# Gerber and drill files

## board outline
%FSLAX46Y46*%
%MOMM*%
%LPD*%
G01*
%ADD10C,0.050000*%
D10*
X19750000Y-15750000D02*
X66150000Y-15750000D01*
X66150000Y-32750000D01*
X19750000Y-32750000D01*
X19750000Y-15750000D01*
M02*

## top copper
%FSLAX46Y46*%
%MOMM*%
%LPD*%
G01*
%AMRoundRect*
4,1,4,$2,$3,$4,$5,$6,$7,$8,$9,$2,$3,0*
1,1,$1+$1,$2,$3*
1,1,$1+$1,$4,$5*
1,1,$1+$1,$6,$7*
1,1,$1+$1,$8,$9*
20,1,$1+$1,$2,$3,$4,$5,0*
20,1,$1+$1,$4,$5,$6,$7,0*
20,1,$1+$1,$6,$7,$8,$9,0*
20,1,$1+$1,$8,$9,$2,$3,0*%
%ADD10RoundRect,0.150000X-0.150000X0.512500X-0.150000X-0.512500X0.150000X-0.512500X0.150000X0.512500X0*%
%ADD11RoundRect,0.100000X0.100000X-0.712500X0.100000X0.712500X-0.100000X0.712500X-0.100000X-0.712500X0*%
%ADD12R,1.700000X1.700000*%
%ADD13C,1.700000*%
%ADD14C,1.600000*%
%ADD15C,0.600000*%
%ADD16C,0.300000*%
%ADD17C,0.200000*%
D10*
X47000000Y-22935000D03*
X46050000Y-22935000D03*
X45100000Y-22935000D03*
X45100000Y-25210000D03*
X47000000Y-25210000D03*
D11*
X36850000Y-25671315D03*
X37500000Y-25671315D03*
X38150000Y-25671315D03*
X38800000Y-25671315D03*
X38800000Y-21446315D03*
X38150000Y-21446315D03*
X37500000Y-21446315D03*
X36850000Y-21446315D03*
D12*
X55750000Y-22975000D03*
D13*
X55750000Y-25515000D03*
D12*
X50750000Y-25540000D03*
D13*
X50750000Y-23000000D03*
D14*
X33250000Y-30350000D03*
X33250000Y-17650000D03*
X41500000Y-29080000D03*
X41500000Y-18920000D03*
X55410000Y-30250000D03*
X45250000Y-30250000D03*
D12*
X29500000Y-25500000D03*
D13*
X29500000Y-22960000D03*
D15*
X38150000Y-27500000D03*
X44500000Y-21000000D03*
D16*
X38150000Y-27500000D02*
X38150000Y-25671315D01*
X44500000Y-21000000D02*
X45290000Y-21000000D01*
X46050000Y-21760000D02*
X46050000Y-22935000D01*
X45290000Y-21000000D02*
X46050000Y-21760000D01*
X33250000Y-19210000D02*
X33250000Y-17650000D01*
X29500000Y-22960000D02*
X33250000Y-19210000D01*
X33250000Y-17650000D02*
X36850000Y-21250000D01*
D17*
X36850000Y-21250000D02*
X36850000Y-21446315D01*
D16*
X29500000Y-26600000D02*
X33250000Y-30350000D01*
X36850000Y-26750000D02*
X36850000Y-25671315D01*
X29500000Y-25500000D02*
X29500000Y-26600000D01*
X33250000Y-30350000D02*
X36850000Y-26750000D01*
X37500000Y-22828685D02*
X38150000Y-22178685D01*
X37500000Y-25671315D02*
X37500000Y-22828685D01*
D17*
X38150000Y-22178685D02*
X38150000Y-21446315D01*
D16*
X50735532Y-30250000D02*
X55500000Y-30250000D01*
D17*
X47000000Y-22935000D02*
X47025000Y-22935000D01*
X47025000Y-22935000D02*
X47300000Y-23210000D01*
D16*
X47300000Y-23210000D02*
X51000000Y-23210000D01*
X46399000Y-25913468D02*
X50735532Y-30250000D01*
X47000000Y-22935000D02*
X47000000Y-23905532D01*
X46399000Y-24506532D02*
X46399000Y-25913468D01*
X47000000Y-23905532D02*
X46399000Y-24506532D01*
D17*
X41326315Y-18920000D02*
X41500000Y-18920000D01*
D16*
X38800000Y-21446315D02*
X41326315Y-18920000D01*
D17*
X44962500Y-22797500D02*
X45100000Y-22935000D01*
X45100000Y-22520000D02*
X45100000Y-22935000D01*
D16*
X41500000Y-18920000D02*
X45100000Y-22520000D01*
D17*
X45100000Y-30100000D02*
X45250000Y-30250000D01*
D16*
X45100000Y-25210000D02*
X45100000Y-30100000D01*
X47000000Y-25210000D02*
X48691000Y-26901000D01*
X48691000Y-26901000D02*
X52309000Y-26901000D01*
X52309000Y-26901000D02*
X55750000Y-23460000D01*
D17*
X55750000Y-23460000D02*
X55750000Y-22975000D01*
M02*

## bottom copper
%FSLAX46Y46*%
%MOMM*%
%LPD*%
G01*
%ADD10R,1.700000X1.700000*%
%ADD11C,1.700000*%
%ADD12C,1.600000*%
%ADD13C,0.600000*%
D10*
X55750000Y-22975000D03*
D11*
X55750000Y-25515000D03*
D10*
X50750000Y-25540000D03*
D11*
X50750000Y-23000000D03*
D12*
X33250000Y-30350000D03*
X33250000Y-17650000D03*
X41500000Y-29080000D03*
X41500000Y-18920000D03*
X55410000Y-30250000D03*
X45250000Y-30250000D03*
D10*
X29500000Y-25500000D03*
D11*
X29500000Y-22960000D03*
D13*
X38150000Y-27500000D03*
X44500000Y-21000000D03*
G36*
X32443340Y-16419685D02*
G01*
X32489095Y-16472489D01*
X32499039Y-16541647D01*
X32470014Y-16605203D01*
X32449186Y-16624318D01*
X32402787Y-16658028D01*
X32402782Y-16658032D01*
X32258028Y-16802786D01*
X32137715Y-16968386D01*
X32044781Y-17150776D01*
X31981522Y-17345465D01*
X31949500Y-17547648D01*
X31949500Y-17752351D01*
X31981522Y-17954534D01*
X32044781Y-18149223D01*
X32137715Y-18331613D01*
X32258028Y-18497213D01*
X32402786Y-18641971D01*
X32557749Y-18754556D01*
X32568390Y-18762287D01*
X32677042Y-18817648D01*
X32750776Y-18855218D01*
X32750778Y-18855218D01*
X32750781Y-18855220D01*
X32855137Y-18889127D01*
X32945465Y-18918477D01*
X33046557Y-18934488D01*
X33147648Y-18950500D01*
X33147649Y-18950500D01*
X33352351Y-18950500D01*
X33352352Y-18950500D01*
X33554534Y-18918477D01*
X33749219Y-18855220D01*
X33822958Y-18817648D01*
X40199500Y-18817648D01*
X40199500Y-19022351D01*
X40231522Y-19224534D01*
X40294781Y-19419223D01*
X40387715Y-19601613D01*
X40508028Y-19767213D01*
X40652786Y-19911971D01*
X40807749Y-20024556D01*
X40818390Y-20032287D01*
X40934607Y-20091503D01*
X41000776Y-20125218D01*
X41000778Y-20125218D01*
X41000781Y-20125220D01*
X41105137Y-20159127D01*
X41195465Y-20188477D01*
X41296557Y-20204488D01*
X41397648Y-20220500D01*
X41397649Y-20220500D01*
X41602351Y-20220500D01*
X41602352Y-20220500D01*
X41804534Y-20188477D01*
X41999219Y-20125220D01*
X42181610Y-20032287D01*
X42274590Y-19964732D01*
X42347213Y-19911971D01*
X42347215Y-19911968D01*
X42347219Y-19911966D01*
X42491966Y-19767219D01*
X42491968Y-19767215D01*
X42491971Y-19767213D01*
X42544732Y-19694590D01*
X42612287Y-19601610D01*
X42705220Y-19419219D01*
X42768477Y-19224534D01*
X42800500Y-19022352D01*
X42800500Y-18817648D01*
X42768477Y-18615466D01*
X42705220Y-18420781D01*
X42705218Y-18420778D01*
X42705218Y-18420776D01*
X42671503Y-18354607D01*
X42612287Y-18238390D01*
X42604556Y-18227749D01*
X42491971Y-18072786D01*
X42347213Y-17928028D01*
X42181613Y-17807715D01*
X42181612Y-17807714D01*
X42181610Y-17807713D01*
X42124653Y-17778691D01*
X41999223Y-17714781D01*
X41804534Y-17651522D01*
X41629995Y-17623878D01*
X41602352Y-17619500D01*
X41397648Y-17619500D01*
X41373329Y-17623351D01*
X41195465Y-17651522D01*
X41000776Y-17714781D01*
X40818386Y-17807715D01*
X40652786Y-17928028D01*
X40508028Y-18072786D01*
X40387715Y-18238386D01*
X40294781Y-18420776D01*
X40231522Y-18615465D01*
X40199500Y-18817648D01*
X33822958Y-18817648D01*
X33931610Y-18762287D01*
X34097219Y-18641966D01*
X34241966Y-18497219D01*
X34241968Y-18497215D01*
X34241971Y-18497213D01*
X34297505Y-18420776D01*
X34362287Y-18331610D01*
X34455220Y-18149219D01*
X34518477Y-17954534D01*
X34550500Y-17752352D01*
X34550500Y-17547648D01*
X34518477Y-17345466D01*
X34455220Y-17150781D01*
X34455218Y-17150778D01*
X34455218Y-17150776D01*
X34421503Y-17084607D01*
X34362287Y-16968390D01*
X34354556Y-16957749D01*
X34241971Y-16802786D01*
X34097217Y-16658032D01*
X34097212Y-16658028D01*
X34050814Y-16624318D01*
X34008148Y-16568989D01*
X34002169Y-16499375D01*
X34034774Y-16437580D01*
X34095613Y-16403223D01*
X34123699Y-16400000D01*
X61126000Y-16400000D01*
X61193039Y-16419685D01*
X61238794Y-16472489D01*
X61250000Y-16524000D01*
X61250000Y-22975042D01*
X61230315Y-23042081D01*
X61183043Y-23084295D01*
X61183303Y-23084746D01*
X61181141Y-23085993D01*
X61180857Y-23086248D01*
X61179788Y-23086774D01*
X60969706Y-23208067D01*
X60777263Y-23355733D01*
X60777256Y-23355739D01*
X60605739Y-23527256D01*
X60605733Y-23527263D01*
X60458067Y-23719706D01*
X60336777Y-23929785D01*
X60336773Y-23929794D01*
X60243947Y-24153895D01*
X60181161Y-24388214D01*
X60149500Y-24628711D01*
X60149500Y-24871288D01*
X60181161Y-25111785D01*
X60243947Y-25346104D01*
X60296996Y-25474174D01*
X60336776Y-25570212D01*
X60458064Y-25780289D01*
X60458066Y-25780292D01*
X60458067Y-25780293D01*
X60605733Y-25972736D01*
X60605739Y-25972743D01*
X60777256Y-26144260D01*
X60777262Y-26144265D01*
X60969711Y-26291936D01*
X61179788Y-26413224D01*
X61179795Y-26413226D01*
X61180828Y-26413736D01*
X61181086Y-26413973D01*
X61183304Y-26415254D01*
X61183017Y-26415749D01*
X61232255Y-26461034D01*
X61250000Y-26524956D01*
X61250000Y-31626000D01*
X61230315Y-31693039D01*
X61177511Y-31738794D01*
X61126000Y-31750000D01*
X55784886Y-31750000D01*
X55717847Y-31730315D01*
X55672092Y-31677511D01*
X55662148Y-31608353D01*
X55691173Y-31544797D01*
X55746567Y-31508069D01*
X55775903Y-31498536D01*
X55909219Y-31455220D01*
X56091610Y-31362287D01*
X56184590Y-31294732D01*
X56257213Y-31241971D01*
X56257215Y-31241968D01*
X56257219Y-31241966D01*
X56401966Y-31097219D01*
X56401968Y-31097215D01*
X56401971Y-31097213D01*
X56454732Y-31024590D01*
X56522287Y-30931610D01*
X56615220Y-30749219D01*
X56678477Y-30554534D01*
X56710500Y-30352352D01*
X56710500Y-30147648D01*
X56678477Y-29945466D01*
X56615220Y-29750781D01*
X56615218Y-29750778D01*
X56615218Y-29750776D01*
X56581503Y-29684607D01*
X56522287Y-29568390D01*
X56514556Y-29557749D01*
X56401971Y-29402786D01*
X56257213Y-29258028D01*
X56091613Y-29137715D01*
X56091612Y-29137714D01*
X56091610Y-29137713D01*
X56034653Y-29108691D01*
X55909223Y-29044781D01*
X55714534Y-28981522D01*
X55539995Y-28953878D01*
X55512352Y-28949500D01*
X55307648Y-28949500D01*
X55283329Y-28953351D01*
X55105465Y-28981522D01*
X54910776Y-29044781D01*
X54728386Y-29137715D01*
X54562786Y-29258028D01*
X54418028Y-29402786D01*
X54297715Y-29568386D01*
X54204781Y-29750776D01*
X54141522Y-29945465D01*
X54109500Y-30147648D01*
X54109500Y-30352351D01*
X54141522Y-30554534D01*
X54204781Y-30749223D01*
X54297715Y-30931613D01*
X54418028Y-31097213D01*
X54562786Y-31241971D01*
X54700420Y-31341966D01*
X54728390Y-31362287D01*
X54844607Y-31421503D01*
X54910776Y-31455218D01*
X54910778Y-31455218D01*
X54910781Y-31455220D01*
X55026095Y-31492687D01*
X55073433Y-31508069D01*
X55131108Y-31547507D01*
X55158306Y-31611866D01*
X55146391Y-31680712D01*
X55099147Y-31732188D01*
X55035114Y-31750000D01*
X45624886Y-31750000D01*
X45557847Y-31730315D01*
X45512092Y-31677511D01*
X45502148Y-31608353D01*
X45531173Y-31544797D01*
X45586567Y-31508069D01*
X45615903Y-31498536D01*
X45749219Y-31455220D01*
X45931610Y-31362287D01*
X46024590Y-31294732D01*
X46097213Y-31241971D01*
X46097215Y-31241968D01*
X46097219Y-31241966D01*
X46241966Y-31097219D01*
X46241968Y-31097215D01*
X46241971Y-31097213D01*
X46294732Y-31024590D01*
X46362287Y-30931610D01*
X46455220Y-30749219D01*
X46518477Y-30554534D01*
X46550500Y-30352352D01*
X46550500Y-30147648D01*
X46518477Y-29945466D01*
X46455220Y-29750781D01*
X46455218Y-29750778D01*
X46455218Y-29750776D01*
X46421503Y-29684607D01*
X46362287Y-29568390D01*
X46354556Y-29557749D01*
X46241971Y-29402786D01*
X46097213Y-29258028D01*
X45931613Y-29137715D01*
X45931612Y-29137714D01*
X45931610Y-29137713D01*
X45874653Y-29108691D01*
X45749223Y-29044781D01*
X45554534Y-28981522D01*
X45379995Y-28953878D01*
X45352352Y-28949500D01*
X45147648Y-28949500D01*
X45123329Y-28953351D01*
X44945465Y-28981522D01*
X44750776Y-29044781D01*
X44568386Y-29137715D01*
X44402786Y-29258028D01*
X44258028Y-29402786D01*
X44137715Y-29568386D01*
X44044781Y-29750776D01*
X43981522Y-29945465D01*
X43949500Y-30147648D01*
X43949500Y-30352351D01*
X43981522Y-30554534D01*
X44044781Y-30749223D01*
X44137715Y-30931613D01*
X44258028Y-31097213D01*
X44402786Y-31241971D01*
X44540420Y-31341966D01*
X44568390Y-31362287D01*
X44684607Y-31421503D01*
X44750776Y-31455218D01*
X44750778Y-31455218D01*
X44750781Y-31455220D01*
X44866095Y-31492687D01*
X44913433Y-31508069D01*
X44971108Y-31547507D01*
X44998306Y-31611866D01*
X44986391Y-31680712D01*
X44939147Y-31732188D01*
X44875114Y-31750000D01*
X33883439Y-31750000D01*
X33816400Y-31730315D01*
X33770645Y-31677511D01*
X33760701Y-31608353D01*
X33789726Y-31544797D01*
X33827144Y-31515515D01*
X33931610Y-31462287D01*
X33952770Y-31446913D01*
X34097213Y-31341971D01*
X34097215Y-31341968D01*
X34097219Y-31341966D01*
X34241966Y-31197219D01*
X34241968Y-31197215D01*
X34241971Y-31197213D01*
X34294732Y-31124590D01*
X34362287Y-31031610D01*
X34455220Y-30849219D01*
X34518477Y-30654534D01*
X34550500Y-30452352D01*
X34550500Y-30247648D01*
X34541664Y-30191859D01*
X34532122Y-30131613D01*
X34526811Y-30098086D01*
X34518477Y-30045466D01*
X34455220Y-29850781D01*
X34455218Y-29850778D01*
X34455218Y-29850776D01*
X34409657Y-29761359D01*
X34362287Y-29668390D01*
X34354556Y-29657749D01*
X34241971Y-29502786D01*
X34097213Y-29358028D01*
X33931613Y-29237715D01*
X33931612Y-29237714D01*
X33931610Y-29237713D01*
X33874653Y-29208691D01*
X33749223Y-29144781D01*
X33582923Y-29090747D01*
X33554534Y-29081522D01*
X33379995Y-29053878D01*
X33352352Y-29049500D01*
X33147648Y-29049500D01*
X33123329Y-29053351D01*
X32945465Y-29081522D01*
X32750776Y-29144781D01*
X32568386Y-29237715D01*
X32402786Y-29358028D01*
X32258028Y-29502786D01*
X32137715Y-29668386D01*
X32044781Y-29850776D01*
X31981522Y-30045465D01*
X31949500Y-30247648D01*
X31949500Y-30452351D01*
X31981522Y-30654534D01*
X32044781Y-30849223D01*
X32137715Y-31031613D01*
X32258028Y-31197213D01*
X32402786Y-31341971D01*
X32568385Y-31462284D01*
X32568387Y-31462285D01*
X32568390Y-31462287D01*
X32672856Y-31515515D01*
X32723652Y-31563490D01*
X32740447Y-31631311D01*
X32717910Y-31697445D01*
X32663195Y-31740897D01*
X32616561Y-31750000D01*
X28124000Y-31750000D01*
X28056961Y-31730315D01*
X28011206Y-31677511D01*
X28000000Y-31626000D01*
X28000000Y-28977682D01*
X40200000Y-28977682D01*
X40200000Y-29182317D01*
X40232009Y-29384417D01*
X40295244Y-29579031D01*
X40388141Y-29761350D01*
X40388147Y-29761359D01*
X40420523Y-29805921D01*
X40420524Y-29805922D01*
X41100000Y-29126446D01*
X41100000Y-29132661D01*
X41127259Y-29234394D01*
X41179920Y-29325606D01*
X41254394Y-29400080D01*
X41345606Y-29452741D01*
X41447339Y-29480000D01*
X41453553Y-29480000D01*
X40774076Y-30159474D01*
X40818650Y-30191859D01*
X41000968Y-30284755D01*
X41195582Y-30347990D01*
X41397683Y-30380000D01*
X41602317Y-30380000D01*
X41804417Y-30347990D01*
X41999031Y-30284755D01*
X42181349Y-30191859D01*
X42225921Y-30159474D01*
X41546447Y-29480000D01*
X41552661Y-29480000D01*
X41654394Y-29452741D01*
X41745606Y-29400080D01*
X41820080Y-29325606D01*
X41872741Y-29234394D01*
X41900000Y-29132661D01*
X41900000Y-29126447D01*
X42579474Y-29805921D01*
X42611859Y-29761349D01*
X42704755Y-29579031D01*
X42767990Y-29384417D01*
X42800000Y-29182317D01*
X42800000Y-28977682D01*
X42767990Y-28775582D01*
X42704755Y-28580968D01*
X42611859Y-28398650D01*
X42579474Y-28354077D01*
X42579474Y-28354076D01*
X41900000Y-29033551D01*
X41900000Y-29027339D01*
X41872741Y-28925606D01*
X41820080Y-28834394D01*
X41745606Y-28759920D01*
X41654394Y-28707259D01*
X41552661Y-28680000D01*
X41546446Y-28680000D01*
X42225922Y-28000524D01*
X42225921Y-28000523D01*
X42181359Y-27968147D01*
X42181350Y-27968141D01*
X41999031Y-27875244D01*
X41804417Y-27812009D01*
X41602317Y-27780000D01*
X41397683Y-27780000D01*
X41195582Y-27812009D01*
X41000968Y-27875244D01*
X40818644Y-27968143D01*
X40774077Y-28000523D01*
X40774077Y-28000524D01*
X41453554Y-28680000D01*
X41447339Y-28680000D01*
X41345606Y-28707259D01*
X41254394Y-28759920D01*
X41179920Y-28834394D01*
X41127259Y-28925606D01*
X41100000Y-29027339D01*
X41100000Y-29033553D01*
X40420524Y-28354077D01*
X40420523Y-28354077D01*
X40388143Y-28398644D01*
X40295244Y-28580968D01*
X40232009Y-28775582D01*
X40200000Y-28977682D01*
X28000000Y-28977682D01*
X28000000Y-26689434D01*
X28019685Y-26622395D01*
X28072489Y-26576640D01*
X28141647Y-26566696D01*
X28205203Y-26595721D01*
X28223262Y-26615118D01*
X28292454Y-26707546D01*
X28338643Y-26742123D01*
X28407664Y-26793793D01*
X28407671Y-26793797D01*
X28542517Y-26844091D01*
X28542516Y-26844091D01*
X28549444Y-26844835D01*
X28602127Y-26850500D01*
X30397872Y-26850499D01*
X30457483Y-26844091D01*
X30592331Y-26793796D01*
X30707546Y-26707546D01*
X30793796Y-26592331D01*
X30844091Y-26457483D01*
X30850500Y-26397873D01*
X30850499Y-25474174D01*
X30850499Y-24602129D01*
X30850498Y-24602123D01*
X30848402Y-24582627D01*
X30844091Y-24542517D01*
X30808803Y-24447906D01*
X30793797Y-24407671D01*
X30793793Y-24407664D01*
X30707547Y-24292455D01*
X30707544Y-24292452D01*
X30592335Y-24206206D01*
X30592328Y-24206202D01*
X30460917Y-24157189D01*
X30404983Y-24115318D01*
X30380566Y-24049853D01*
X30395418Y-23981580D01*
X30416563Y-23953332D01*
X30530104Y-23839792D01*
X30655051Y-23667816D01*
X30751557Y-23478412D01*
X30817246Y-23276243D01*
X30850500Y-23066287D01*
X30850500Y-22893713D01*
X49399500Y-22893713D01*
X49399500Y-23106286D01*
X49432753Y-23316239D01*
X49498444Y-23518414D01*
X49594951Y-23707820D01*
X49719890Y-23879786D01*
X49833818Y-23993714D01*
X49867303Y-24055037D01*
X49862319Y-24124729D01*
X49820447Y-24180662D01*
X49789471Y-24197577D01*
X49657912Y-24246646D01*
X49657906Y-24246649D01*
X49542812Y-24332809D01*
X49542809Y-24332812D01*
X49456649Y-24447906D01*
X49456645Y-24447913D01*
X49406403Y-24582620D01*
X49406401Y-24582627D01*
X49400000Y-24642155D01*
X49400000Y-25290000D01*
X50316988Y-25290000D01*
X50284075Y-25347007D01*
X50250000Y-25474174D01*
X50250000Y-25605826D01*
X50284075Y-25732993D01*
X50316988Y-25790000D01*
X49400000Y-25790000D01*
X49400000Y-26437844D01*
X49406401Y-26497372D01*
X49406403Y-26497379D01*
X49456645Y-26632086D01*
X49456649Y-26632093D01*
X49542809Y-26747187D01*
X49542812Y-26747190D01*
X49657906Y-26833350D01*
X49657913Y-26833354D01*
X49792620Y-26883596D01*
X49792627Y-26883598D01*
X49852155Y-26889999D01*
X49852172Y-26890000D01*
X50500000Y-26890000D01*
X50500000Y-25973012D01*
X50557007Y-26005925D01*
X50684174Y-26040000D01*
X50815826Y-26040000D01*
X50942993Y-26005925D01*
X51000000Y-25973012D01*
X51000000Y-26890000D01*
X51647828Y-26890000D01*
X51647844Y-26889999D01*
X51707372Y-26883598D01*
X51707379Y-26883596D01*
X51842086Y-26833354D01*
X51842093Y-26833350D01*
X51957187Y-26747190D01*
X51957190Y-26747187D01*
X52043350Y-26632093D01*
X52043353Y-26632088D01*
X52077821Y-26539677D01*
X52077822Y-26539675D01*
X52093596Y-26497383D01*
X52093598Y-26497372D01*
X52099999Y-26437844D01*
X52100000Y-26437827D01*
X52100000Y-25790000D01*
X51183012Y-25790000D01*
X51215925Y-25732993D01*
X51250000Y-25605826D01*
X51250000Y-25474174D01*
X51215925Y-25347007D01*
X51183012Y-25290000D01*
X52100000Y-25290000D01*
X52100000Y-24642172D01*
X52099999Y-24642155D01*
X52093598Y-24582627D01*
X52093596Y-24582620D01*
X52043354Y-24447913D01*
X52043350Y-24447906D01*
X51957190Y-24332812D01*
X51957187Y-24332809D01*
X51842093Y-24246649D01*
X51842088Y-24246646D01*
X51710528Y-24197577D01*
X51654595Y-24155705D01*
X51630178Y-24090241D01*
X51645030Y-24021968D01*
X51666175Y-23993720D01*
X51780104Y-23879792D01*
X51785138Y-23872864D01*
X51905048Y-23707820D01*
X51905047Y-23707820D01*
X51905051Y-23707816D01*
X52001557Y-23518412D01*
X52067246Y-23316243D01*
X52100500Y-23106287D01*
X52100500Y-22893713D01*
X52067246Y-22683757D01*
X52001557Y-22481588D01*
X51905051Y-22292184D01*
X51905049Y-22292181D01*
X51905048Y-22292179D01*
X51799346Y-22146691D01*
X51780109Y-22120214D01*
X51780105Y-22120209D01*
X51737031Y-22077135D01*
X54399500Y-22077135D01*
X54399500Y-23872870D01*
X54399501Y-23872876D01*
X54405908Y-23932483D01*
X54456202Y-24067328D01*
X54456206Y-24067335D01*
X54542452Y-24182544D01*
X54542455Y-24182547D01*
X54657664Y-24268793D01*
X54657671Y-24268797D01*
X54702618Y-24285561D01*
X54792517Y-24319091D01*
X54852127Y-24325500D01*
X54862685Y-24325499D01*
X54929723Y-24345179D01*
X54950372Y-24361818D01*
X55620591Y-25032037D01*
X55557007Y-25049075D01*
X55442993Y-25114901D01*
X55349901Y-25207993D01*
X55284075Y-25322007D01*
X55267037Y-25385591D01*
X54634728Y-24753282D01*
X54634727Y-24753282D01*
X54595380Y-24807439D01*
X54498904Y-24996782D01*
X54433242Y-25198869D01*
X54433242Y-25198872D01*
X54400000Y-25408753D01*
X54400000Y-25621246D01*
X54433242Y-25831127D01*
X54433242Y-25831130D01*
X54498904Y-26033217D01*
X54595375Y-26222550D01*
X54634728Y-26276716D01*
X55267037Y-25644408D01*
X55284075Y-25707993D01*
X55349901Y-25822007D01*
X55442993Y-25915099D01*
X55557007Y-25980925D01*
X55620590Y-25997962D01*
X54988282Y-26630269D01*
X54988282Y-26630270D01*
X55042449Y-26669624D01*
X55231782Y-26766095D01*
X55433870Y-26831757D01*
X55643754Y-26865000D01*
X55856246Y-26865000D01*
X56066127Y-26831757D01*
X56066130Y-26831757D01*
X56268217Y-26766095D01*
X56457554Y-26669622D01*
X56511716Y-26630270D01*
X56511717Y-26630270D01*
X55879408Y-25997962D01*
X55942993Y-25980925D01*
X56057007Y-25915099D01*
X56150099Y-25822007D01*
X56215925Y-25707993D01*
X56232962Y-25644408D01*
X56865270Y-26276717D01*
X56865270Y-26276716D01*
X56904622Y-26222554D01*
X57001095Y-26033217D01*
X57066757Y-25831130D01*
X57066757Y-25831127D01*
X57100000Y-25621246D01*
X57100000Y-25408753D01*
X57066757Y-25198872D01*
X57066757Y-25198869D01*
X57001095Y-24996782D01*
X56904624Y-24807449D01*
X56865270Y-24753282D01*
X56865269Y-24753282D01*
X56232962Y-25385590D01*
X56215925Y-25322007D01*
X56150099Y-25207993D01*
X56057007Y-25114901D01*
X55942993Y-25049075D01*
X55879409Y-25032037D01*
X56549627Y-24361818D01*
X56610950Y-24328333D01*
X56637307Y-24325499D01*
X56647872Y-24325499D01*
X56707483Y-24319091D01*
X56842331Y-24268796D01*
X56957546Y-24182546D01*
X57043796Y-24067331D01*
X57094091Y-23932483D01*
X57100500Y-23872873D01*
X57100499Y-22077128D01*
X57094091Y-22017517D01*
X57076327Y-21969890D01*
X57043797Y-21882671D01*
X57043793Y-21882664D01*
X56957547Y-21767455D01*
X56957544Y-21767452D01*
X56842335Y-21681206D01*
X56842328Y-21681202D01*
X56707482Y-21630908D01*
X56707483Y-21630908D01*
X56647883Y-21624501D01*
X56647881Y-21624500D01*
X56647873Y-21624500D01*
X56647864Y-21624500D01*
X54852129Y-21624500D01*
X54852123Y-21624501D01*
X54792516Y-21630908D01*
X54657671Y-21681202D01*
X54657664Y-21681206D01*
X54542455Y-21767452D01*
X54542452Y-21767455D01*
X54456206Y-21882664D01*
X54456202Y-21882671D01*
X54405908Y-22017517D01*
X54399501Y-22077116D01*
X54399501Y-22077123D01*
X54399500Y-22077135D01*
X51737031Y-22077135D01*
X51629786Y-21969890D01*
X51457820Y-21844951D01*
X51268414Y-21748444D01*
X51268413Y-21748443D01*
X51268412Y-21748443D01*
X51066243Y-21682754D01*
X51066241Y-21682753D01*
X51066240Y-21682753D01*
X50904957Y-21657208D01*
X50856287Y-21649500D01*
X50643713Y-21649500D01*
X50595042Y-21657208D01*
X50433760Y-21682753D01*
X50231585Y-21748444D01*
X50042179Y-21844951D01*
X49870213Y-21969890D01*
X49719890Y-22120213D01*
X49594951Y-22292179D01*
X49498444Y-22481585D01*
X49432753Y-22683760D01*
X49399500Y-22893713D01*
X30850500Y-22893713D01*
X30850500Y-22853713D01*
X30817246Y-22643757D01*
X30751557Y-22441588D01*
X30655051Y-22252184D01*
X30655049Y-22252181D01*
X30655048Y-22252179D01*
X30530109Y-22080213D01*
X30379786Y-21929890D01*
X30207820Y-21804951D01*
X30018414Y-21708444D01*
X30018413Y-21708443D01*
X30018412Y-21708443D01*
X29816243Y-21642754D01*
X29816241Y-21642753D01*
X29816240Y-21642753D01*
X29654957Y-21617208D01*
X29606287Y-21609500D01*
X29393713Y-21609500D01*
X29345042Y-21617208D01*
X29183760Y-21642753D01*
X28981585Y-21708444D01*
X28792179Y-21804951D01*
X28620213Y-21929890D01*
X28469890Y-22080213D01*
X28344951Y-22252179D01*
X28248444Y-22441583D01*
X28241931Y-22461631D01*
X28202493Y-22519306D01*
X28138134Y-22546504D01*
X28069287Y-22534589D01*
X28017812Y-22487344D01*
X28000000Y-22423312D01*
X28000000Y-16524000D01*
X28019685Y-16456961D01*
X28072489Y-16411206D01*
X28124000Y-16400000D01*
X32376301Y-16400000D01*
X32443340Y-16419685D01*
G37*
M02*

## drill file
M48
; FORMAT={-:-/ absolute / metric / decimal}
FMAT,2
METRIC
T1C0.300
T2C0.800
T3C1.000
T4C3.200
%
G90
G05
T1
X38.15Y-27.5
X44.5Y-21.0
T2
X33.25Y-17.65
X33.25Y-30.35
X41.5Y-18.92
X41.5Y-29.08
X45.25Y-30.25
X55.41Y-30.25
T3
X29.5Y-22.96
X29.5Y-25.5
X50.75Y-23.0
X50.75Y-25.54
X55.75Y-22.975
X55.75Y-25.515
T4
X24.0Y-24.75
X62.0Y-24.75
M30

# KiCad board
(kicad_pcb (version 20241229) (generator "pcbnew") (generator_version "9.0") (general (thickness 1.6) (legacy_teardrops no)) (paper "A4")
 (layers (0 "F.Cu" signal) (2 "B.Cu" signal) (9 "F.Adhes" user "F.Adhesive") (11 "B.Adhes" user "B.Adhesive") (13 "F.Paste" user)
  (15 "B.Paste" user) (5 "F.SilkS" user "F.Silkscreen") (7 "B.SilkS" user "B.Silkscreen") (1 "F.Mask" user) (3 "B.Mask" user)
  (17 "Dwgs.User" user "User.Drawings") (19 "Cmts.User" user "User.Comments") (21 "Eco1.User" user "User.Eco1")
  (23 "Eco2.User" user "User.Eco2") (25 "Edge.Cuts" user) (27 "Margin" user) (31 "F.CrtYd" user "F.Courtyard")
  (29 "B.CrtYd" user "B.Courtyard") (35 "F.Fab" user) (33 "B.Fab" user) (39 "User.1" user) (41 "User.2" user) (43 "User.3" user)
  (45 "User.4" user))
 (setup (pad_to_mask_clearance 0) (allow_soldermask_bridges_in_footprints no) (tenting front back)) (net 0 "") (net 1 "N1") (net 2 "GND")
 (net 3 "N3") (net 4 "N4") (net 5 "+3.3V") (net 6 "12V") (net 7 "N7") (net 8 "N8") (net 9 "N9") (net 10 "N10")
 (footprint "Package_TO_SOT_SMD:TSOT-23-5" (layer "F.Cu") (at 46.05 24.0725 -90)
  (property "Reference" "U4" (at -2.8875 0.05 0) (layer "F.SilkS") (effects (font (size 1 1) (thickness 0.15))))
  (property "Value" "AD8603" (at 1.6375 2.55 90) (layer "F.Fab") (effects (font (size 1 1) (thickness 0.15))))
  (pad "1" smd roundrect (at -1.1375 -0.95 270) (size 1.325 0.6) (layers "F.Cu" "F.Mask" "F.Paste") (roundrect_rratio 0.25) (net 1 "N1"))
  (pad "2" smd roundrect (at -1.1375 0 270) (size 1.325 0.6) (layers "F.Cu" "F.Mask" "F.Paste") (roundrect_rratio 0.25) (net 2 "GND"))
  (pad "3" smd roundrect (at -1.1375 0.95 270) (size 1.325 0.6) (layers "F.Cu" "F.Mask" "F.Paste") (roundrect_rratio 0.25) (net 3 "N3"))
  (pad "4" smd roundrect (at 1.1375 0.95 270) (size 1.325 0.6) (layers "F.Cu" "F.Mask" "F.Paste") (roundrect_rratio 0.25) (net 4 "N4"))
  (pad "5" smd roundrect (at 1.1375 -0.95 270) (size 1.325 0.6) (layers "F.Cu" "F.Mask" "F.Paste") (roundrect_rratio 0.25) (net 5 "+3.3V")))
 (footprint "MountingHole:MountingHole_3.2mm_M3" (layer "F.Cu") (at 62 24.75)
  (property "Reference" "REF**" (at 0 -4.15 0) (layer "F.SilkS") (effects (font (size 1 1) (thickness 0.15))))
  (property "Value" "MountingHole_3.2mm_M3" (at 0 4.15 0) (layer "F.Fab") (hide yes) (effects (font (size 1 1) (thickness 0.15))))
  (pad "" np_thru_hole circle (at 0 0) (size 3.2 3.2) (drill 3.2) (layers "*.Cu" "*.Mask")))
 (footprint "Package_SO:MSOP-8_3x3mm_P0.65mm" (layer "F.Cu") (at 37.825 23.558815 90)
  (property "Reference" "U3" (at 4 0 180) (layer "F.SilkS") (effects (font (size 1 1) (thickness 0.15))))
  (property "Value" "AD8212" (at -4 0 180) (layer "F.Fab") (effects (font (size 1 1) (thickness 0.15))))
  (pad "1" smd roundrect (at -2.1125 -0.975 90) (size 1.625 0.4) (layers "F.Cu" "F.Mask" "F.Paste") (roundrect_rratio 0.25) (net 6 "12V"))
  (pad "2" smd roundrect (at -2.1125 -0.325 90) (size 1.625 0.4) (layers "F.Cu" "F.Mask" "F.Paste") (roundrect_rratio 0.25) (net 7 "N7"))
  (pad "3" smd roundrect (at -2.1125 0.325 90) (size 1.625 0.4) (layers "F.Cu" "F.Mask" "F.Paste") (roundrect_rratio 0.25) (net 2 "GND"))
  (pad "4" smd roundrect (at -2.1125 0.975 90) (size 1.625 0.4) (layers "F.Cu" "F.Mask" "F.Paste") (roundrect_rratio 0.25) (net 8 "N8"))
  (pad "5" smd roundrect (at 2.1125 0.975 90) (size 1.625 0.4) (layers "F.Cu" "F.Mask" "F.Paste") (roundrect_rratio 0.25) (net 3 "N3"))
  (pad "6" smd roundrect (at 2.1125 0.325 90) (size 1.625 0.4) (layers "F.Cu" "F.Mask" "F.Paste") (roundrect_rratio 0.25) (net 7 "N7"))
  (pad "7" smd roundrect (at 2.1125 -0.325 90) (size 1.625 0.4) (layers "F.Cu" "F.Mask" "F.Paste") (roundrect_rratio 0.25) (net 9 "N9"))
  (pad "8" smd roundrect (at 2.1125 -0.975 90) (size 1.625 0.4) (layers "F.Cu" "F.Mask" "F.Paste") (roundrect_rratio 0.25) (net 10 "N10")))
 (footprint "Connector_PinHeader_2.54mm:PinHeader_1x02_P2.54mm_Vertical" (layer "F.Cu") (at 55.75 22.975)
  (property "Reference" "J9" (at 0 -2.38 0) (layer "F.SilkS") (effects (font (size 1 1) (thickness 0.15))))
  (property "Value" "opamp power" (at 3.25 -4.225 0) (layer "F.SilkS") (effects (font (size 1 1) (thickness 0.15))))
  (pad "1" thru_hole rect (at 0 0) (size 1.7 1.7) (drill 1) (layers "*.Cu" "*.Mask") (remove_unused_layers no) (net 5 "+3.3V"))
  (pad "2" thru_hole circle (at 0 2.54) (size 1.7 1.7) (drill 1) (layers "*.Cu" "*.Mask") (remove_unused_layers no) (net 2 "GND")))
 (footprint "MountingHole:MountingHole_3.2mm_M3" (layer "F.Cu") (at 24 24.75)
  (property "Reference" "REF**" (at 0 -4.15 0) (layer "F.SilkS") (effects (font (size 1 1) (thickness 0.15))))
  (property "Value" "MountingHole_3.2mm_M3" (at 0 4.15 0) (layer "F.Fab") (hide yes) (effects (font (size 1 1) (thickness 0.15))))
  (pad "" np_thru_hole circle (at 0 0) (size 3.2 3.2) (drill 3.2) (layers "*.Cu" "*.Mask")))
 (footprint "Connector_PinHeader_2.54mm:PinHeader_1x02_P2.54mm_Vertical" (layer "F.Cu") (at 50.75 25.54 180)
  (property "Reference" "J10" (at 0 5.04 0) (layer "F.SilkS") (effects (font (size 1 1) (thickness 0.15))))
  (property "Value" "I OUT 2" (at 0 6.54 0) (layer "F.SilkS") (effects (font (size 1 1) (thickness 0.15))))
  (pad "1" thru_hole rect (at 0 0 180) (size 1.7 1.7) (drill 1) (layers "*.Cu" "*.Mask") (remove_unused_layers no) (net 2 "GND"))
  (pad "2" thru_hole circle (at 0 2.54 180) (size 1.7 1.7) (drill 1) (layers "*.Cu" "*.Mask") (remove_unused_layers no) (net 1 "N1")))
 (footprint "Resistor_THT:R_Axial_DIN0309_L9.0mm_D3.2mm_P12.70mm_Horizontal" (layer "F.Cu") (at 33.25 30.35 90)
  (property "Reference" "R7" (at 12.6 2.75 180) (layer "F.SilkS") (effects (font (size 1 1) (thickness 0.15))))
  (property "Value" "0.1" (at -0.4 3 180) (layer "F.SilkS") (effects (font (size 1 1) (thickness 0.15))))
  (pad "1" thru_hole circle (at 0 0 90) (size 1.6 1.6) (drill 0.8) (layers "*.Cu" "*.Mask") (remove_unused_layers no) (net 6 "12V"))
  (pad "2" thru_hole circle (at 12.7 0 90) (size 1.6 1.6) (drill 0.8) (layers "*.Cu" "*.Mask") (remove_unused_layers no) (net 10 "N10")))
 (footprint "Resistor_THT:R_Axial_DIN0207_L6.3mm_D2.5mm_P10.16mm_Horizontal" (layer "F.Cu") (at 41.5 29.08 90)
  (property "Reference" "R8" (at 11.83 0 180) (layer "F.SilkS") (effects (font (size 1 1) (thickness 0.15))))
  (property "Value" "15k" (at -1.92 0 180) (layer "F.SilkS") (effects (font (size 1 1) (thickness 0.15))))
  (pad "1" thru_hole circle (at 0 0 90) (size 1.6 1.6) (drill 0.8) (layers "*.Cu" "*.Mask") (remove_unused_layers no) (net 2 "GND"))
  (pad "2" thru_hole circle (at 10.16 0 90) (size 1.6 1.6) (drill 0.8) (layers "*.Cu" "*.Mask") (remove_unused_layers no) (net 3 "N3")))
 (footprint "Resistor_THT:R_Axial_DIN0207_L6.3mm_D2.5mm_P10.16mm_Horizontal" (layer "F.Cu") (at 55.41 30.25 180)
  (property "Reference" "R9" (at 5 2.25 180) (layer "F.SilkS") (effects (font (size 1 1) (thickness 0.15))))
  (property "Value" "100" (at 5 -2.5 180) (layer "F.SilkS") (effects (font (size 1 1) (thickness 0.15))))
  (pad "1" thru_hole circle (at 0 0 180) (size 1.6 1.6) (drill 0.8) (layers "*.Cu" "*.Mask") (remove_unused_layers no) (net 1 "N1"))
  (pad "2" thru_hole circle (at 10.16 0 180) (size 1.6 1.6) (drill 0.8) (layers "*.Cu" "*.Mask") (remove_unused_layers no) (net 4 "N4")))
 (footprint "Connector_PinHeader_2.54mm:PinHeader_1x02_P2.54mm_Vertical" (layer "F.Cu") (at 29.5 25.5 180)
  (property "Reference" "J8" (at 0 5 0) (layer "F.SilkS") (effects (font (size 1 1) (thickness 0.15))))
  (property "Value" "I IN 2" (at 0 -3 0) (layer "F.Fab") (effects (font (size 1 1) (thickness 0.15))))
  (pad "1" thru_hole rect (at 0 0 180) (size 1.7 1.7) (drill 1) (layers "*.Cu" "*.Mask") (remove_unused_layers no) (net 6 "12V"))
  (pad "2" thru_hole circle (at 0 2.54 180) (size 1.7 1.7) (drill 1) (layers "*.Cu" "*.Mask") (remove_unused_layers no) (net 10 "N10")))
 (gr_rect (start 19.75 15.75) (end 66.15 32.75) (stroke (width 0.05) (type default)) (fill no) (layer "Edge.Cuts"))
 (segment (start 38.15 27.5) (end 38.15 25.671315) (width 0.3) (layer "F.Cu") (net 2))
 (segment (start 44.5 21) (end 45.29 21) (width 0.3) (layer "F.Cu") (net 2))
 (segment (start 46.05 21.76) (end 46.05 22.935) (width 0.3) (layer "F.Cu") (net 2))
 (segment (start 45.29 21) (end 46.05 21.76) (width 0.3) (layer "F.Cu") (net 2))
 (via (at 38.15 27.5) (size 0.6) (drill 0.3) (layers "F.Cu" "B.Cu") (free yes) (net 2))
 (via (at 44.5 21) (size 0.6) (drill 0.3) (layers "F.Cu" "B.Cu") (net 2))
 (segment (start 33.25 19.21) (end 33.25 17.65) (width 0.3) (layer "F.Cu") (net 10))
 (segment (start 29.5 22.96) (end 33.25 19.21) (width 0.3) (layer "F.Cu") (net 10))
 (segment (start 33.25 17.65) (end 36.85 21.25) (width 0.3) (layer "F.Cu") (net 10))
 (segment (start 36.85 21.25) (end 36.85 21.446315) (width 0.2) (layer "F.Cu") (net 10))
 (segment (start 29.5 26.6) (end 33.25 30.35) (width 0.3) (layer "F.Cu") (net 6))
 (segment (start 36.85 26.75) (end 36.85 25.671315) (width 0.3) (layer "F.Cu") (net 6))
 (segment (start 29.5 25.5) (end 29.5 26.6) (width 0.3) (layer "F.Cu") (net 6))
 (segment (start 33.25 30.35) (end 36.85 26.75) (width 0.3) (layer "F.Cu") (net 6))
 (segment (start 37.5 22.828685) (end 38.15 22.178685) (width 0.3) (layer "F.Cu") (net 7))
 (segment (start 37.5 25.671315) (end 37.5 22.828685) (width 0.3) (layer "F.Cu") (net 7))
 (segment (start 38.15 22.178685) (end 38.15 21.446315) (width 0.2) (layer "F.Cu") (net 7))
 (segment (start 50.735532 30.25) (end 55.5 30.25) (width 0.3) (layer "F.Cu") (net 1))
 (segment (start 47 22.935) (end 47.025 22.935) (width 0.2) (layer "F.Cu") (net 1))
 (segment (start 47.025 22.935) (end 47.3 23.21) (width 0.2) (layer "F.Cu") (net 1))
 (segment (start 47.3 23.21) (end 51 23.21) (width 0.3) (layer "F.Cu") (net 1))
 (segment (start 46.399 25.913468) (end 50.735532 30.25) (width 0.3) (layer "F.Cu") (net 1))
 (segment (start 47 22.935) (end 47 23.905532) (width 0.3) (layer "F.Cu") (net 1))
 (segment (start 46.399 24.506532) (end 46.399 25.913468) (width 0.3) (layer "F.Cu") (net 1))
 (segment (start 47 23.905532) (end 46.399 24.506532) (width 0.3) (layer "F.Cu") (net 1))
 (segment (start 41.326315 18.92) (end 41.5 18.92) (width 0.2) (layer "F.Cu") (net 3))
 (segment (start 38.8 21.446315) (end 41.326315 18.92) (width 0.3) (layer "F.Cu") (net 3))
 (segment (start 44.9625 22.7975) (end 45.1 22.935) (width 0.2) (layer "F.Cu") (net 3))
 (segment (start 45.1 22.52) (end 45.1 22.935) (width 0.2) (layer "F.Cu") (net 3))
 (segment (start 41.5 18.92) (end 45.1 22.52) (width 0.3) (layer "F.Cu") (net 3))
 (segment (start 45.1 30.1) (end 45.25 30.25) (width 0.2) (layer "F.Cu") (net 4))
 (segment (start 45.1 25.21) (end 45.1 30.1) (width 0.3) (layer "F.Cu") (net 4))
 (segment (start 47 25.21) (end 48.691 26.901) (width 0.3) (layer "F.Cu") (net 5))
 (segment (start 48.691 26.901) (end 52.309 26.901) (width 0.3) (layer "F.Cu") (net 5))
 (segment (start 52.309 26.901) (end 55.75 23.46) (width 0.3) (layer "F.Cu") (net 5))
 (segment (start 55.75 23.46) (end 55.75 22.975) (width 0.2) (layer "F.Cu") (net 5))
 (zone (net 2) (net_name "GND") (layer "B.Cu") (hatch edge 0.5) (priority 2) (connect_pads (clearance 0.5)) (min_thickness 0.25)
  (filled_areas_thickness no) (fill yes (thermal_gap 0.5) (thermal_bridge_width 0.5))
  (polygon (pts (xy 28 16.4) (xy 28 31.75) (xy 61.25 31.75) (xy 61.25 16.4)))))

